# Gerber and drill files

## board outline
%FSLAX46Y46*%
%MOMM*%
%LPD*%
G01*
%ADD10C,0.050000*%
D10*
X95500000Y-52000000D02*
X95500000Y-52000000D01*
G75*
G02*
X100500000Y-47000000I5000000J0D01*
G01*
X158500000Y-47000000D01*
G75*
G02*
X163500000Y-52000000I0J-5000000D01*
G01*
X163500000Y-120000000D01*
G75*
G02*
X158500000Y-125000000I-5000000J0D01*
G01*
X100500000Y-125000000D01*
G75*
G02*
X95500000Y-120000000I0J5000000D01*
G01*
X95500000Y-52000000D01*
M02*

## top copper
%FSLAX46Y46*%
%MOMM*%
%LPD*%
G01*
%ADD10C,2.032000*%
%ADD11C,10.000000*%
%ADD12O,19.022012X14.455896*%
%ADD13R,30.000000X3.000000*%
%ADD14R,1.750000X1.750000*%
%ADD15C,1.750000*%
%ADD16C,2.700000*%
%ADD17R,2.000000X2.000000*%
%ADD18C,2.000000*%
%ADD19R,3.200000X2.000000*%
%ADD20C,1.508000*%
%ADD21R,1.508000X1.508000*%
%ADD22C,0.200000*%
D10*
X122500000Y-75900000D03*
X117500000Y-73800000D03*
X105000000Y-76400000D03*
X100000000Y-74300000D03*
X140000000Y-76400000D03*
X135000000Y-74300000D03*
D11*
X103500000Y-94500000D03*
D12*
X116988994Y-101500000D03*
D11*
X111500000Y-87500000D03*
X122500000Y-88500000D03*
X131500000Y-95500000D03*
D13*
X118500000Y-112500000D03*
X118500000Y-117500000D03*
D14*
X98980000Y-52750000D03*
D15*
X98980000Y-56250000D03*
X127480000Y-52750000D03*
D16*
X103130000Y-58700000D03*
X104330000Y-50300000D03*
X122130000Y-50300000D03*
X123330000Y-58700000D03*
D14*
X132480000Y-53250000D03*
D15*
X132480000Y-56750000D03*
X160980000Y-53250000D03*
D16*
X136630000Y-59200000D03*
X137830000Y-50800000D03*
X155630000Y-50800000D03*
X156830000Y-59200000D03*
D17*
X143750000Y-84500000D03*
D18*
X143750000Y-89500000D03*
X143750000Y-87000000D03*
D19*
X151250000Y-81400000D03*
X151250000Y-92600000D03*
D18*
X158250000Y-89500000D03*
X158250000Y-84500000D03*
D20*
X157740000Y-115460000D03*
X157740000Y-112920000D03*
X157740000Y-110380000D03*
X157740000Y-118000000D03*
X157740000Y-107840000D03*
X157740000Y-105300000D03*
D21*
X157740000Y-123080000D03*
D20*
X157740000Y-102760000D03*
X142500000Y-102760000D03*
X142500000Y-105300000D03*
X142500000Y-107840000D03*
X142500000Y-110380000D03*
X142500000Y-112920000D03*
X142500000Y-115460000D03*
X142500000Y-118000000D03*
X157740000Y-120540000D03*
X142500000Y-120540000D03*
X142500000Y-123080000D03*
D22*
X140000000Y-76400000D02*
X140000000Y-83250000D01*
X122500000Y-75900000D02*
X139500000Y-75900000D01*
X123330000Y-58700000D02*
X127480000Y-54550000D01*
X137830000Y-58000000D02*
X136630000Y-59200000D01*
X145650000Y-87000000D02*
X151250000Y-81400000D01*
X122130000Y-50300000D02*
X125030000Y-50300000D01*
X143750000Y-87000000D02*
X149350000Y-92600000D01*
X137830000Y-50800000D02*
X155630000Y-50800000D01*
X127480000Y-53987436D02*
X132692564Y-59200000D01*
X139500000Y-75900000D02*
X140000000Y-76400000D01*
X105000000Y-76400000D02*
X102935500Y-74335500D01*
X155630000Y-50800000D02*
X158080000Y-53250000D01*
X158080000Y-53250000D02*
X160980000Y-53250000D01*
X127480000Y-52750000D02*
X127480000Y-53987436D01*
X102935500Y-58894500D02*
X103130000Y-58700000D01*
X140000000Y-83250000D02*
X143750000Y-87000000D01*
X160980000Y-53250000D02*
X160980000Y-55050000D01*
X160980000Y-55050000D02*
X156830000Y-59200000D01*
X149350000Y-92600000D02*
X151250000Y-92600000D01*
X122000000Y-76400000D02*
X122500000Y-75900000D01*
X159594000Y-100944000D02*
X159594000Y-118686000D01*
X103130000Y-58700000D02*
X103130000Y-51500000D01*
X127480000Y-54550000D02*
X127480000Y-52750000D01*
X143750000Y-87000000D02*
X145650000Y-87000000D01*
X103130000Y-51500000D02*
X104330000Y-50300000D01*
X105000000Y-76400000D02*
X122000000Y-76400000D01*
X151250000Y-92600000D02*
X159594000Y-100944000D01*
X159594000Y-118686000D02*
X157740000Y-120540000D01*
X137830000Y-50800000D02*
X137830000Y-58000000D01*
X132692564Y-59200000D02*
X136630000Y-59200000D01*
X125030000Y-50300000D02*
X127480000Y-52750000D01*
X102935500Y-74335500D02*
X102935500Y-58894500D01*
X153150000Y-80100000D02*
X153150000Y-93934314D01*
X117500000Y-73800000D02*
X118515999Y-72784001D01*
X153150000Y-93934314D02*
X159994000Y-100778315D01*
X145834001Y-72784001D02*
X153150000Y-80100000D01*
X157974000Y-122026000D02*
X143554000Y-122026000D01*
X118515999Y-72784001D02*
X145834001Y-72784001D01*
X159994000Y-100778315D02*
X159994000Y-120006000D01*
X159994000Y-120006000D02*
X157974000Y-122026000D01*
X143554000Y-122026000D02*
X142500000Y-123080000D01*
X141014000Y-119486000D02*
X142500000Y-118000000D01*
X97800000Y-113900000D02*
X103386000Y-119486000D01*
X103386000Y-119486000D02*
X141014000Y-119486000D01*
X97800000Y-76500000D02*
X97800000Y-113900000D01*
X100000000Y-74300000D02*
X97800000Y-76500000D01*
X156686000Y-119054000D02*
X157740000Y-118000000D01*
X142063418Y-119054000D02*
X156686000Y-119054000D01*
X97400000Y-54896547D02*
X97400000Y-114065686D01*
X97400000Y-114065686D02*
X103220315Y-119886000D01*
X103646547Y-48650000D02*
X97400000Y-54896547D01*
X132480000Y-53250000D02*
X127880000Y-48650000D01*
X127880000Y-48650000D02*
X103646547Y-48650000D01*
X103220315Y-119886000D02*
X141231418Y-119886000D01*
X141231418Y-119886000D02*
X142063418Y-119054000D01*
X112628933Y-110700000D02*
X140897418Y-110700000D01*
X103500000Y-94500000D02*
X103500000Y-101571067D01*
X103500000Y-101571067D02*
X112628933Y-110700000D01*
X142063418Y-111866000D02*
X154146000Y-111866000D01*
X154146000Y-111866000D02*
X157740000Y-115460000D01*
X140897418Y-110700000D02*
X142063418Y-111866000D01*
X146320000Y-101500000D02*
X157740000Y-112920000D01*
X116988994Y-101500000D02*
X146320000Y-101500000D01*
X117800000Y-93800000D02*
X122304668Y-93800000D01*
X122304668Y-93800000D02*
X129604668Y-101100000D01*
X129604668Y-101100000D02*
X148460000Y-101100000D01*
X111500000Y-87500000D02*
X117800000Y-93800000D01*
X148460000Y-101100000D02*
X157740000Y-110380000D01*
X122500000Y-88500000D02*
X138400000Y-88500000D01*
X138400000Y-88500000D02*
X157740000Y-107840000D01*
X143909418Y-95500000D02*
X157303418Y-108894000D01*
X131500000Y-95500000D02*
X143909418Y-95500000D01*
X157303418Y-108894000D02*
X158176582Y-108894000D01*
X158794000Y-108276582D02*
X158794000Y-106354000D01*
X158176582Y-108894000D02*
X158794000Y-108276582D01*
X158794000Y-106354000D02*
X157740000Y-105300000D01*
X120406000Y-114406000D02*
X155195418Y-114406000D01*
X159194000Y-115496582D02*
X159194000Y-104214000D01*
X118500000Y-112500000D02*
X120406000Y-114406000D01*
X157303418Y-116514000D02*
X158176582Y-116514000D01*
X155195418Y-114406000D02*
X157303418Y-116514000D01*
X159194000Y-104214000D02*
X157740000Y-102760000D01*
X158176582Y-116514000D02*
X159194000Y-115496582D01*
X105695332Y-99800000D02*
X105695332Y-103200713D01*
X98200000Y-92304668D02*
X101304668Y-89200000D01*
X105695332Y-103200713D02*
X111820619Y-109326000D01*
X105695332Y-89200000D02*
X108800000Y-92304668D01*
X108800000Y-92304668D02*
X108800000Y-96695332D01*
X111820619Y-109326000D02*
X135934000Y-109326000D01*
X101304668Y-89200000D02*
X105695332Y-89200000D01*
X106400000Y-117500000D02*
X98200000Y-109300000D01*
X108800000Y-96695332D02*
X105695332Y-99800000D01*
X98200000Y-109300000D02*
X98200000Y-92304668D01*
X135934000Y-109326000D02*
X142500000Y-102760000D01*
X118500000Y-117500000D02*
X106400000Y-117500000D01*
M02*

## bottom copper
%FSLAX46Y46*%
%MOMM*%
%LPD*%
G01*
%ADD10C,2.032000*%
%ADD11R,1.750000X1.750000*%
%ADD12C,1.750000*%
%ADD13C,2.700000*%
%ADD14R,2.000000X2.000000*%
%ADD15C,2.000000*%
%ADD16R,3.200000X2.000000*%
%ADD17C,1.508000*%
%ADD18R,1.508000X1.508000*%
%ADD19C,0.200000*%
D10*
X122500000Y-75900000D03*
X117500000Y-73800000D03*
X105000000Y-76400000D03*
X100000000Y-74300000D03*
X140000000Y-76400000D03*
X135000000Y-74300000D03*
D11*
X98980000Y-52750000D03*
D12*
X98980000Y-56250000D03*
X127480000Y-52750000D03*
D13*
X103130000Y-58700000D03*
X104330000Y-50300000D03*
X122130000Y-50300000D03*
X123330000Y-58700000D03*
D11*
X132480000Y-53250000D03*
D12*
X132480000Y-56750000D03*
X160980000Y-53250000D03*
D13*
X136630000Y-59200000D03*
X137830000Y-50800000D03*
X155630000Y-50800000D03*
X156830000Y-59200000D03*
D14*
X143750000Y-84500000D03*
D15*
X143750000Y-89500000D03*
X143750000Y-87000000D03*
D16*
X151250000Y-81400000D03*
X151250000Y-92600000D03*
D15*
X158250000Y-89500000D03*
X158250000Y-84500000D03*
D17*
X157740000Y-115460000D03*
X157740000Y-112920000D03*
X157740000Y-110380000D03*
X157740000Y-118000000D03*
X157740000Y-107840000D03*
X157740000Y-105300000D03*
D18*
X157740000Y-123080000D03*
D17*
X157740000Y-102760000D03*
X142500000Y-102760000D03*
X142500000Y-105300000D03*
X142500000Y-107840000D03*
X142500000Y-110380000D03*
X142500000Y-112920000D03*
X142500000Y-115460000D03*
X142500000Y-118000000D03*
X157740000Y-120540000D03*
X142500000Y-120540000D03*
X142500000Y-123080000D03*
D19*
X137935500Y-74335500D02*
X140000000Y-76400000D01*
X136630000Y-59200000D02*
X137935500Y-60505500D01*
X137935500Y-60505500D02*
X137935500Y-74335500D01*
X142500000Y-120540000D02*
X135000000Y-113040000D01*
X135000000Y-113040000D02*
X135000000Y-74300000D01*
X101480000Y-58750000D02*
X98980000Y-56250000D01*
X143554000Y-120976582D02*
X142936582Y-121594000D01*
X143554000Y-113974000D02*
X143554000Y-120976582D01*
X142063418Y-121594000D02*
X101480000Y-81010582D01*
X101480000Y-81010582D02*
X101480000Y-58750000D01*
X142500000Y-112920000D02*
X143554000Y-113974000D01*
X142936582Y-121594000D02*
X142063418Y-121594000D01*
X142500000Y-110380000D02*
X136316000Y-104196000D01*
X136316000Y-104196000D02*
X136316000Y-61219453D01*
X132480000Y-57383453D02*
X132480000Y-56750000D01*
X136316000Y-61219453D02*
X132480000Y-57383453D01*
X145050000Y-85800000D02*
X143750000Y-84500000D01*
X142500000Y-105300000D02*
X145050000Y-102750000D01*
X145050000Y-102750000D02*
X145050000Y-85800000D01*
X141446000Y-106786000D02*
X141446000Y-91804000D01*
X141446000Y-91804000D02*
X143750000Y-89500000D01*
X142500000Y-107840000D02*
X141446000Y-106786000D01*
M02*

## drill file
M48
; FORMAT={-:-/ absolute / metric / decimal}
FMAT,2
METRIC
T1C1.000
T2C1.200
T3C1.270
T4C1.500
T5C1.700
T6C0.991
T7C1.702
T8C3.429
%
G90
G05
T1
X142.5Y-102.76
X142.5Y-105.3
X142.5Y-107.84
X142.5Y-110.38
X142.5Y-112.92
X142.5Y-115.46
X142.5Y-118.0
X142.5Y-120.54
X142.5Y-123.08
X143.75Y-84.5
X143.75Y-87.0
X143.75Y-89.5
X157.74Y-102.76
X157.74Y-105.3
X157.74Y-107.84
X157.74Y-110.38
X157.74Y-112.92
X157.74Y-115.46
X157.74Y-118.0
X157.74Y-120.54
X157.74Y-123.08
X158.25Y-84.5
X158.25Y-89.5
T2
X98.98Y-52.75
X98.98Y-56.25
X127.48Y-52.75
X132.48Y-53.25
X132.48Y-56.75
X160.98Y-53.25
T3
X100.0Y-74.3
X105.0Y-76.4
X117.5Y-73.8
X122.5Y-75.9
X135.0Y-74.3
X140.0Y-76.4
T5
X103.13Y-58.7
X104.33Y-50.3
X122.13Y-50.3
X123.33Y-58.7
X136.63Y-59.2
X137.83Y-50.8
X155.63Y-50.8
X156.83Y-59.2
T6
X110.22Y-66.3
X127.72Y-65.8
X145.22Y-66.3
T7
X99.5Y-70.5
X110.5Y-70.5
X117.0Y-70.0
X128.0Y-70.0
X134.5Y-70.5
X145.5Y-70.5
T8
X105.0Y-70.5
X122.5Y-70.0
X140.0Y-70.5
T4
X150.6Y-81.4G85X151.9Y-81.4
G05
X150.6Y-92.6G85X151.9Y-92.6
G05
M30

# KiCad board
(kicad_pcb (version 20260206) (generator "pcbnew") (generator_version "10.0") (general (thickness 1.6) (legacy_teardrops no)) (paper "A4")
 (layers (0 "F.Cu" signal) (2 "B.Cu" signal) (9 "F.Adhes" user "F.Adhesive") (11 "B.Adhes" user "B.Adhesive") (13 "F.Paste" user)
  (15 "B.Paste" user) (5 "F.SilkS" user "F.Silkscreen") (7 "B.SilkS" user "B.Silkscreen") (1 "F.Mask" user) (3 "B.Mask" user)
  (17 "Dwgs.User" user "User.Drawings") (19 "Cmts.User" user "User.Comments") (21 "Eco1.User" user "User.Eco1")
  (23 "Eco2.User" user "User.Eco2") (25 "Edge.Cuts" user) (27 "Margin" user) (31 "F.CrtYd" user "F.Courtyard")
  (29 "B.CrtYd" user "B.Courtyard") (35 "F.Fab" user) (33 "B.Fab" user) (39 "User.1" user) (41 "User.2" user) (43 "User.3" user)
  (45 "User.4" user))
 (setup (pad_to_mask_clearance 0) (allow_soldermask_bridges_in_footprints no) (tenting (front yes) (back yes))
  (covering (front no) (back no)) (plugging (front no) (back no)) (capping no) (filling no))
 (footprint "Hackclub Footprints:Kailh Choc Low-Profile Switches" (layer "F.Cu") (at 122.5 70)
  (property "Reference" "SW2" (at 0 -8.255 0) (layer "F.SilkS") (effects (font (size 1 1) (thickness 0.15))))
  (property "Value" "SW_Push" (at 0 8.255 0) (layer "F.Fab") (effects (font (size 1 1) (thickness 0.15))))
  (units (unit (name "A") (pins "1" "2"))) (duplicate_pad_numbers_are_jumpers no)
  (pad "" np_thru_hole circle (at -5.5 0) (size 1.7018 1.7018) (drill 1.7018) (layers "*.Cu" "*.Mask"))
  (pad "" np_thru_hole circle (at 0 0) (size 3.429 3.429) (drill 3.429) (layers "*.Cu" "*.Mask"))
  (pad "" np_thru_hole circle (at 5.22 -4.2) (size 0.9906 0.9906) (drill 0.9906) (layers "*.Cu" "*.Mask"))
  (pad "" np_thru_hole circle (at 5.5 0) (size 1.7018 1.7018) (drill 1.7018) (layers "*.Cu" "*.Mask"))
  (pad "1" thru_hole circle (at 0 5.9) (size 2.032 2.032) (drill 1.27) (layers "*.Cu" "*.Mask") (remove_unused_layers no) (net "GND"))
  (pad "2" thru_hole circle (at -5 3.8) (size 2.032 2.032) (drill 1.27) (layers "*.Cu" "*.Mask") (remove_unused_layers no) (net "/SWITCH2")))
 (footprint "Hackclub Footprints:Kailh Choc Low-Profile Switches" (layer "F.Cu") (at 105 70.5)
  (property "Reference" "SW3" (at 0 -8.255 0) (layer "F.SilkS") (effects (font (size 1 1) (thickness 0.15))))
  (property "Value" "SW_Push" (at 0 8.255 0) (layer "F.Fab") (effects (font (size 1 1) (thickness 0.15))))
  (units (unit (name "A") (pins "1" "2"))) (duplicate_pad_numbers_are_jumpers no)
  (pad "" np_thru_hole circle (at -5.5 0) (size 1.7018 1.7018) (drill 1.7018) (layers "*.Cu" "*.Mask"))
  (pad "" np_thru_hole circle (at 0 0) (size 3.429 3.429) (drill 3.429) (layers "*.Cu" "*.Mask"))
  (pad "" np_thru_hole circle (at 5.22 -4.2) (size 0.9906 0.9906) (drill 0.9906) (layers "*.Cu" "*.Mask"))
  (pad "" np_thru_hole circle (at 5.5 0) (size 1.7018 1.7018) (drill 1.7018) (layers "*.Cu" "*.Mask"))
  (pad "1" thru_hole circle (at 0 5.9) (size 2.032 2.032) (drill 1.27) (layers "*.Cu" "*.Mask") (remove_unused_layers no) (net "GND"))
  (pad "2" thru_hole circle (at -5 3.8) (size 2.032 2.032) (drill 1.27) (layers "*.Cu" "*.Mask") (remove_unused_layers no) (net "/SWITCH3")))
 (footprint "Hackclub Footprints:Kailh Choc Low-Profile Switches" (layer "F.Cu") (at 140 70.5)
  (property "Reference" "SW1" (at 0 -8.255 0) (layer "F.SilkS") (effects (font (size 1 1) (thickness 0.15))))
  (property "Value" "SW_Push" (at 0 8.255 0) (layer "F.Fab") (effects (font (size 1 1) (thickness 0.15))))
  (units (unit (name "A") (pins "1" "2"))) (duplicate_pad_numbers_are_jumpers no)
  (pad "" np_thru_hole circle (at -5.5 0) (size 1.7018 1.7018) (drill 1.7018) (layers "*.Cu" "*.Mask"))
  (pad "" np_thru_hole circle (at 0 0) (size 3.429 3.429) (drill 3.429) (layers "*.Cu" "*.Mask"))
  (pad "" np_thru_hole circle (at 5.22 -4.2) (size 0.9906 0.9906) (drill 0.9906) (layers "*.Cu" "*.Mask"))
  (pad "" np_thru_hole circle (at 5.5 0) (size 1.7018 1.7018) (drill 1.7018) (layers "*.Cu" "*.Mask"))
  (pad "1" thru_hole circle (at 0 5.9) (size 2.032 2.032) (drill 1.27) (layers "*.Cu" "*.Mask") (remove_unused_layers no) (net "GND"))
  (pad "2" thru_hole circle (at -5 3.8) (size 2.032 2.032) (drill 1.27) (layers "*.Cu" "*.Mask") (remove_unused_layers no) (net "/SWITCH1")))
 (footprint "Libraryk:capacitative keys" (layer "F.Cu") (at 102.5 54.5)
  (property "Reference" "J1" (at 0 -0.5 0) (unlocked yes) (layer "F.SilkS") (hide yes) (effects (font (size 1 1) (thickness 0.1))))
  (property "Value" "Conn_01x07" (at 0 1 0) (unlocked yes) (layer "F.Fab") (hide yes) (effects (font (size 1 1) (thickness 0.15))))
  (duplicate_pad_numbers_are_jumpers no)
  (pad "1" smd circle (at 1 40) (size 10 10) (layers "F.Cu" "F.Mask") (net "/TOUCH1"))
  (pad "2" smd oval (at 14.488994 47 90) (size 14.455896 19.022012) (layers "F.Cu" "F.Mask") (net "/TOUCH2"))
  (pad "3" smd circle (at 9 33) (size 10 10) (layers "F.Cu" "F.Mask") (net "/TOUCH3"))
  (pad "4" smd circle (at 20 34) (size 10 10) (layers "F.Cu" "F.Mask") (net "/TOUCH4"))
  (pad "5" smd circle (at 29 41) (size 10 10) (layers "F.Cu" "F.Mask") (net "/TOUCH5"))
  (pad "6" smd rect (at 16 58) (size 30 3) (layers "F.Cu" "F.Mask") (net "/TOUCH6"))
  (pad "7" smd rect (at 16 63) (size 30 3) (layers "F.Cu" "F.Mask") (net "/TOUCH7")))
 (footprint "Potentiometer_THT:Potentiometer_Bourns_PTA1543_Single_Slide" (layer "F.Cu") (at 98.98 52.75)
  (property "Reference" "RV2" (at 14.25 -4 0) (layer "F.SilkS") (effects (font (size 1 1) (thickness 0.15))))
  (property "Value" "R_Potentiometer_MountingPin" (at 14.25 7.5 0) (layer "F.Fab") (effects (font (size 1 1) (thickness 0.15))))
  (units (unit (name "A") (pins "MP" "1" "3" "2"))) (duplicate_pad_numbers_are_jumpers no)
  (pad "1" thru_hole rect (at 0 0) (size 1.75 1.75) (drill 1.2) (layers "*.Cu" "*.Mask") (remove_unused_layers no) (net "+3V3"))
  (pad "2" thru_hole circle (at 0 3.5) (size 1.75 1.75) (drill 1.2) (layers "*.Cu" "*.Mask") (remove_unused_layers no) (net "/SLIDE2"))
  (pad "3" thru_hole circle (at 28.5 0) (size 1.75 1.75) (drill 1.2) (layers "*.Cu" "*.Mask") (remove_unused_layers no) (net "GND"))
  (pad "MP" thru_hole circle (at 4.15 5.95) (size 2.7 2.7) (drill 1.7) (layers "*.Cu" "*.Mask") (remove_unused_layers no) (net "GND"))
  (pad "MP" thru_hole circle (at 5.35 -2.45) (size 2.7 2.7) (drill 1.7) (layers "*.Cu" "*.Mask") (remove_unused_layers no) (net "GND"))
  (pad "MP" thru_hole circle (at 23.15 -2.45) (size 2.7 2.7) (drill 1.7) (layers "*.Cu" "*.Mask") (remove_unused_layers no) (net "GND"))
  (pad "MP" thru_hole circle (at 24.35 5.95) (size 2.7 2.7) (drill 1.7) (layers "*.Cu" "*.Mask") (remove_unused_layers no) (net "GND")))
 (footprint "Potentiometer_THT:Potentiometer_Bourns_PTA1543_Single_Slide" (layer "F.Cu") (at 132.48 53.25)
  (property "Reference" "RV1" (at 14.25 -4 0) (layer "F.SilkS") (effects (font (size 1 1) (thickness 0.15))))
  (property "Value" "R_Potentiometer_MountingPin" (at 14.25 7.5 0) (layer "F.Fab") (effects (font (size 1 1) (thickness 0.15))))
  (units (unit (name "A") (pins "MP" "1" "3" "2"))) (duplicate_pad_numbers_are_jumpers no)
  (pad "1" thru_hole rect (at 0 0) (size 1.75 1.75) (drill 1.2) (layers "*.Cu" "*.Mask") (remove_unused_layers no) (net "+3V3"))
  (pad "2" thru_hole circle (at 0 3.5) (size 1.75 1.75) (drill 1.2) (layers "*.Cu" "*.Mask") (remove_unused_layers no) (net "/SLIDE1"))
  (pad "3" thru_hole circle (at 28.5 0) (size 1.75 1.75) (drill 1.2) (layers "*.Cu" "*.Mask") (remove_unused_layers no) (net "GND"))
  (pad "MP" thru_hole circle (at 4.15 5.95) (size 2.7 2.7) (drill 1.7) (layers "*.Cu" "*.Mask") (remove_unused_layers no) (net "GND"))
  (pad "MP" thru_hole circle (at 5.35 -2.45) (size 2.7 2.7) (drill 1.7) (layers "*.Cu" "*.Mask") (remove_unused_layers no) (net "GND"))
  (pad "MP" thru_hole circle (at 23.15 -2.45) (size 2.7 2.7) (drill 1.7) (layers "*.Cu" "*.Mask") (remove_unused_layers no) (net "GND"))
  (pad "MP" thru_hole circle (at 24.35 5.95) (size 2.7 2.7) (drill 1.7) (layers "*.Cu" "*.Mask") (remove_unused_layers no) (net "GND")))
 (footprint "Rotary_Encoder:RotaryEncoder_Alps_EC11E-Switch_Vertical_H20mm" (layer "F.Cu") (at 143.75 84.5)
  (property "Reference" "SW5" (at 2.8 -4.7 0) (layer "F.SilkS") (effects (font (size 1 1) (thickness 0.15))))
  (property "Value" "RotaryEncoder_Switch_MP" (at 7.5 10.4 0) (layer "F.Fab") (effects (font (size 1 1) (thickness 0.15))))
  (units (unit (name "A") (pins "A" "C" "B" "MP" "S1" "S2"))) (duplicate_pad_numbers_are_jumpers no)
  (pad "A" thru_hole rect (at 0 0) (size 2 2) (drill 1) (layers "*.Cu" "*.Mask") (remove_unused_layers no) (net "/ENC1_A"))
  (pad "B" thru_hole circle (at 0 5) (size 2 2) (drill 1) (layers "*.Cu" "*.Mask") (remove_unused_layers no) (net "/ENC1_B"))
  (pad "C" thru_hole circle (at 0 2.5) (size 2 2) (drill 1) (layers "*.Cu" "*.Mask") (remove_unused_layers no) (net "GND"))
  (pad "MP" thru_hole rect (at 7.5 -3.1) (size 3.2 2) (drill oval 2.8 1.5) (layers "*.Cu" "*.Mask") (remove_unused_layers no) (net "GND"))
  (pad "MP" thru_hole rect (at 7.5 8.1) (size 3.2 2) (drill oval 2.8 1.5) (layers "*.Cu" "*.Mask") (remove_unused_layers no) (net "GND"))
  (pad "S1" thru_hole circle (at 14.5 5) (size 2 2) (drill 1) (layers "*.Cu" "*.Mask") (remove_unused_layers no)
   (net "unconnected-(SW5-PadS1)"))
  (pad "S2" thru_hole circle (at 14.5 0) (size 2 2) (drill 1) (layers "*.Cu" "*.Mask") (remove_unused_layers no)
   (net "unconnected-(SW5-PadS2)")))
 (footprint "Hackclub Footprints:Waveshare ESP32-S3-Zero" (layer "F.Cu") (at 150.12 112.92 180)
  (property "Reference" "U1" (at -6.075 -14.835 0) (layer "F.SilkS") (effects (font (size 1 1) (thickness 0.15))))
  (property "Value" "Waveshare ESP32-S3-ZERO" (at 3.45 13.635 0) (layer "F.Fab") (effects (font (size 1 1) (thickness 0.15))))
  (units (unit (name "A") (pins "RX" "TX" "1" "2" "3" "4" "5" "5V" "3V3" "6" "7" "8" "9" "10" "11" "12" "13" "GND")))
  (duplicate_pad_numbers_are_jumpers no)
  (pad "1" thru_hole circle (at -7.62 -2.54 180) (size 1.508 1.508) (drill 1) (layers "*.Cu" "*.Mask") (remove_unused_layers no)
   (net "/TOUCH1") (solder_mask_margin 0.102))
  (pad "2" thru_hole circle (at -7.62 0 180) (size 1.508 1.508) (drill 1) (layers "*.Cu" "*.Mask") (remove_unused_layers no) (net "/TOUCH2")
   (solder_mask_margin 0.102))
  (pad "3" thru_hole circle (at -7.62 2.54 180) (size 1.508 1.508) (drill 1) (layers "*.Cu" "*.Mask") (remove_unused_layers no)
   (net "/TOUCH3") (solder_mask_margin 0.102))
  (pad "3V3" thru_hole circle (at -7.62 -5.08 180) (size 1.508 1.508) (drill 1) (layers "*.Cu" "*.Mask") (remove_unused_layers no)
   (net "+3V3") (solder_mask_margin 0.102))
  (pad "4" thru_hole circle (at -7.62 5.08 180) (size 1.508 1.508) (drill 1) (layers "*.Cu" "*.Mask") (remove_unused_layers no)
   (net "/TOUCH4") (solder_mask_margin 0.102))
  (pad "5" thru_hole circle (at -7.62 7.62 180) (size 1.508 1.508) (drill 1) (layers "*.Cu" "*.Mask") (remove_unused_layers no)
   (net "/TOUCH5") (solder_mask_margin 0.102))
  (pad "5V" thru_hole rect (at -7.62 -10.16 180) (size 1.508 1.508) (drill 1) (layers "*.Cu" "*.Mask") (remove_unused_layers no) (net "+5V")
   (solder_mask_margin 0.102))
  (pad "6" thru_hole circle (at -7.62 10.16 180) (size 1.508 1.508) (drill 1) (layers "*.Cu" "*.Mask") (remove_unused_layers no)
   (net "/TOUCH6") (solder_mask_margin 0.102))
  (pad "7" thru_hole circle (at 7.62 10.16 180) (size 1.508 1.508) (drill 1) (layers "*.Cu" "*.Mask") (remove_unused_layers no)
   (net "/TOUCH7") (solder_mask_margin 0.102))
  (pad "8" thru_hole circle (at 7.62 7.62 180) (size 1.508 1.508) (drill 1) (layers "*.Cu" "*.Mask") (remove_unused_layers no)
   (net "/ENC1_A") (solder_mask_margin 0.102))
  (pad "9" thru_hole circle (at 7.62 5.08 180) (size 1.508 1.508) (drill 1) (layers "*.Cu" "*.Mask") (remove_unused_layers no)
   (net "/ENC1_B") (solder_mask_margin 0.102))
  (pad "10" thru_hole circle (at 7.62 2.54 180) (size 1.508 1.508) (drill 1) (layers "*.Cu" "*.Mask") (remove_unused_layers no)
   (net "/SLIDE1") (solder_mask_margin 0.102))
  (pad "11" thru_hole circle (at 7.62 0 180) (size 1.508 1.508) (drill 1) (layers "*.Cu" "*.Mask") (remove_unused_layers no) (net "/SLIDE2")
   (solder_mask_margin 0.102))
  (pad "12" thru_hole circle (at 7.62 -2.54 180) (size 1.508 1.508) (drill 1) (layers "*.Cu" "*.Mask") (remove_unused_layers no)
   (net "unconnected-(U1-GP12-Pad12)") (solder_mask_margin 0.102))
  (pad "13" thru_hole circle (at 7.62 -5.08 180) (size 1.508 1.508) (drill 1) (layers "*.Cu" "*.Mask") (remove_unused_layers no)
   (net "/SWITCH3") (solder_mask_margin 0.102))
  (pad "GND" thru_hole circle (at -7.62 -7.62 180) (size 1.508 1.508) (drill 1) (layers "*.Cu" "*.Mask") (remove_unused_layers no)
   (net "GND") (solder_mask_margin 0.102))
  (pad "RX" thru_hole circle (at 7.62 -7.62 180) (size 1.508 1.508) (drill 1) (layers "*.Cu" "*.Mask") (remove_unused_layers no)
   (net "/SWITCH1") (solder_mask_margin 0.102))
  (pad "TX" thru_hole circle (at 7.62 -10.16 180) (size 1.508 1.508) (drill 1) (layers "*.Cu" "*.Mask") (remove_unused_layers no)
   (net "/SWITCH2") (solder_mask_margin 0.102)))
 (gr_rect (start 95.5 47) (end 163.5 125) (radius 5) (stroke (width 0.05) (type solid)) (fill no) (layer "Edge.Cuts"))
 (segment (start 140 76.4) (end 140 83.25) (width 0.2) (layer "F.Cu") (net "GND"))
 (segment (start 122.5 75.9) (end 139.5 75.9) (width 0.2) (layer "F.Cu") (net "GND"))
 (segment (start 123.33 58.7) (end 127.48 54.55) (width 0.2) (layer "F.Cu") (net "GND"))
 (segment (start 137.83 58) (end 136.63 59.2) (width 0.2) (layer "F.Cu") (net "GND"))
 (segment (start 145.65 87) (end 151.25 81.4) (width 0.2) (layer "F.Cu") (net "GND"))
 (segment (start 122.13 50.3) (end 125.03 50.3) (width 0.2) (layer "F.Cu") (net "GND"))
 (segment (start 143.75 87) (end 149.35 92.6) (width 0.2) (layer "F.Cu") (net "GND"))
 (segment (start 137.83 50.8) (end 155.63 50.8) (width 0.2) (layer "F.Cu") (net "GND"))
 (segment (start 127.48 53.987436) (end 132.692564 59.2) (width 0.2) (layer "F.Cu") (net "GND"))
 (segment (start 139.5 75.9) (end 140 76.4) (width 0.2) (layer "F.Cu") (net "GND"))
 (segment (start 105 76.4) (end 102.9355 74.3355) (width 0.2) (layer "F.Cu") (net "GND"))
 (segment (start 155.63 50.8) (end 158.08 53.25) (width 0.2) (layer "F.Cu") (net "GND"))
 (segment (start 158.08 53.25) (end 160.98 53.25) (width 0.2) (layer "F.Cu") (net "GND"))
 (segment (start 127.48 52.75) (end 127.48 53.987436) (width 0.2) (layer "F.Cu") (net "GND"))
 (segment (start 102.9355 58.8945) (end 103.13 58.7) (width 0.2) (layer "F.Cu") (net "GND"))
 (segment (start 140 83.25) (end 143.75 87) (width 0.2) (layer "F.Cu") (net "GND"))
 (segment (start 160.98 53.25) (end 160.98 55.05) (width 0.2) (layer "F.Cu") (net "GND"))
 (segment (start 160.98 55.05) (end 156.83 59.2) (width 0.2) (layer "F.Cu") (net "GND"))
 (segment (start 149.35 92.6) (end 151.25 92.6) (width 0.2) (layer "F.Cu") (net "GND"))
 (segment (start 122 76.4) (end 122.5 75.9) (width 0.2) (layer "F.Cu") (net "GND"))
 (segment (start 159.594 100.944) (end 159.594 118.686) (width 0.2) (layer "F.Cu") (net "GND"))
 (segment (start 103.13 58.7) (end 103.13 51.5) (width 0.2) (layer "F.Cu") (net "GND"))
 (segment (start 127.48 54.55) (end 127.48 52.75) (width 0.2) (layer "F.Cu") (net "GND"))
 (segment (start 143.75 87) (end 145.65 87) (width 0.2) (layer "F.Cu") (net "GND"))
 (segment (start 103.13 51.5) (end 104.33 50.3) (width 0.2) (layer "F.Cu") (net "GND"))
 (segment (start 105 76.4) (end 122 76.4) (width 0.2) (layer "F.Cu") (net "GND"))
 (segment (start 151.25 92.6) (end 159.594 100.944) (width 0.2) (layer "F.Cu") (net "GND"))
 (segment (start 159.594 118.686) (end 157.74 120.54) (width 0.2) (layer "F.Cu") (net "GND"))
 (segment (start 137.83 50.8) (end 137.83 58) (width 0.2) (layer "F.Cu") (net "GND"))
 (segment (start 132.692564 59.2) (end 136.63 59.2) (width 0.2) (layer "F.Cu") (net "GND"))
 (segment (start 125.03 50.3) (end 127.48 52.75) (width 0.2) (layer "F.Cu") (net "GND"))
 (segment (start 102.9355 74.3355) (end 102.9355 58.8945) (width 0.2) (layer "F.Cu") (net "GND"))
 (segment (start 137.9355 74.3355) (end 140 76.4) (width 0.2) (layer "B.Cu") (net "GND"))
 (segment (start 136.63 59.2) (end 137.9355 60.5055) (width 0.2) (layer "B.Cu") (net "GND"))
 (segment (start 137.9355 60.5055) (end 137.9355 74.3355) (width 0.2) (layer "B.Cu") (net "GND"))
 (segment (start 153.15 80.1) (end 153.15 93.934314) (width 0.2) (layer "F.Cu") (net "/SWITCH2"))
 (segment (start 117.5 73.8) (end 118.515999 72.784001) (width 0.2) (layer "F.Cu") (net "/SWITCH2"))
 (segment (start 153.15 93.934314) (end 159.994 100.778315) (width 0.2) (layer "F.Cu") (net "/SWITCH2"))
 (segment (start 145.834001 72.784001) (end 153.15 80.1) (width 0.2) (layer "F.Cu") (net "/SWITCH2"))
 (segment (start 157.974 122.026) (end 143.554 122.026) (width 0.2) (layer "F.Cu") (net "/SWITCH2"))
 (segment (start 118.515999 72.784001) (end 145.834001 72.784001) (width 0.2) (layer "F.Cu") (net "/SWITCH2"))
 (segment (start 159.994 100.778315) (end 159.994 120.006) (width 0.2) (layer "F.Cu") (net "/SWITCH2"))
 (segment (start 159.994 120.006) (end 157.974 122.026) (width 0.2) (layer "F.Cu") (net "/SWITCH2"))
 (segment (start 143.554 122.026) (end 142.5 123.08) (width 0.2) (layer "F.Cu") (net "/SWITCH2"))
 (segment (start 141.014 119.486) (end 142.5 118) (width 0.2) (layer "F.Cu") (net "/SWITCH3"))
 (segment (start 97.8 113.9) (end 103.386 119.486) (width 0.2) (layer "F.Cu") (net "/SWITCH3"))
 (segment (start 103.386 119.486) (end 141.014 119.486) (width 0.2) (layer "F.Cu") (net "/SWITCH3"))
 (segment (start 97.8 76.5) (end 97.8 113.9) (width 0.2) (layer "F.Cu") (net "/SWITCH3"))
 (segment (start 100 74.3) (end 97.8 76.5) (width 0.2) (layer "F.Cu") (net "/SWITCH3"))
 (segment (start 142.5 120.54) (end 135 113.04) (width 0.2) (layer "B.Cu") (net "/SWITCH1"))
 (segment (start 135 113.04) (end 135 74.3) (width 0.2) (layer "B.Cu") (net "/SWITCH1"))
 (segment (start 156.686 119.054) (end 157.74 118) (width 0.2) (layer "F.Cu") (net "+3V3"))
 (segment (start 142.063418 119.054) (end 156.686 119.054) (width 0.2) (layer "F.Cu") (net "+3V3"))
 (segment (start 97.4 54.896547) (end 97.4 114.065686) (width 0.2) (layer "F.Cu") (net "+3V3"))
 (segment (start 97.4 114.065686) (end 103.220315 119.886) (width 0.2) (layer "F.Cu") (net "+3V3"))
 (segment (start 103.646547 48.65) (end 97.4 54.896547) (width 0.2) (layer "F.Cu") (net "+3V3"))
 (segment (start 132.48 53.25) (end 127.88 48.65) (width 0.2) (layer "F.Cu") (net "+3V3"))
 (segment (start 127.88 48.65) (end 103.646547 48.65) (width 0.2) (layer "F.Cu") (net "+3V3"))
 (segment (start 103.220315 119.886) (end 141.231418 119.886) (width 0.2) (layer "F.Cu") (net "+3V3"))
 (segment (start 141.231418 119.886) (end 142.063418 119.054) (width 0.2) (layer "F.Cu") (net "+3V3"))
 (segment (start 101.48 58.75) (end 98.98 56.25) (width 0.2) (layer "B.Cu") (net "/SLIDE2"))
 (segment (start 143.554 120.976582) (end 142.936582 121.594) (width 0.2) (layer "B.Cu") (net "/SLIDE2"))
 (segment (start 143.554 113.974) (end 143.554 120.976582) (width 0.2) (layer "B.Cu") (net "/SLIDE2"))
 (segment (start 142.063418 121.594) (end 101.48 81.010582) (width 0.2) (layer "B.Cu") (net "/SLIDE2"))
 (segment (start 101.48 81.010582) (end 101.48 58.75) (width 0.2) (layer "B.Cu") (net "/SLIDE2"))
 (segment (start 142.5 112.92) (end 143.554 113.974) (width 0.2) (layer "B.Cu") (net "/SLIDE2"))
 (segment (start 142.936582 121.594) (end 142.063418 121.594) (width 0.2) (layer "B.Cu") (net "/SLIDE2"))
 (segment (start 142.5 110.38) (end 136.316 104.196) (width 0.2) (layer "B.Cu") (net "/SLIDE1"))
 (segment (start 136.316 104.196) (end 136.316 61.219453) (width 0.2) (layer "B.Cu") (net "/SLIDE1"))
 (segment (start 132.48 57.383453) (end 132.48 56.75) (width 0.2) (layer "B.Cu") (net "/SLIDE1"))
 (segment (start 136.316 61.219453) (end 132.48 57.383453) (width 0.2) (layer "B.Cu") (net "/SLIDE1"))
 (segment (start 145.05 85.8) (end 143.75 84.5) (width 0.2) (layer "B.Cu") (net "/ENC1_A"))
 (segment (start 142.5 105.3) (end 145.05 102.75) (width 0.2) (layer "B.Cu") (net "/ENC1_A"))
 (segment (start 145.05 102.75) (end 145.05 85.8) (width 0.2) (layer "B.Cu") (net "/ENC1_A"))
 (segment (start 141.446 106.786) (end 141.446 91.804) (width 0.2) (layer "B.Cu") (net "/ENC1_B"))
 (segment (start 141.446 91.804) (end 143.75 89.5) (width 0.2) (layer "B.Cu") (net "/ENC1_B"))
 (segment (start 142.5 107.84) (end 141.446 106.786) (width 0.2) (layer "B.Cu") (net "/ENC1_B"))
 (segment (start 112.628933 110.7) (end 140.897418 110.7) (width 0.2) (layer "F.Cu") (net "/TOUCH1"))
 (segment (start 103.5 94.5) (end 103.5 101.571067) (width 0.2) (layer "F.Cu") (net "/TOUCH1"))
 (segment (start 103.5 101.571067) (end 112.628933 110.7) (width 0.2) (layer "F.Cu") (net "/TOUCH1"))
 (segment (start 142.063418 111.866) (end 154.146 111.866) (width 0.2) (layer "F.Cu") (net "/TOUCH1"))
 (segment (start 154.146 111.866) (end 157.74 115.46) (width 0.2) (layer "F.Cu") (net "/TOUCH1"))
 (segment (start 140.897418 110.7) (end 142.063418 111.866) (width 0.2) (layer "F.Cu") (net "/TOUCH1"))
 (segment (start 146.32 101.5) (end 157.74 112.92) (width 0.2) (layer "F.Cu") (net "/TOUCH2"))
 (segment (start 116.988994 101.5) (end 146.32 101.5) (width 0.2) (layer "F.Cu") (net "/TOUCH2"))
 (segment (start 117.8 93.8) (end 122.304668 93.8) (width 0.2) (layer "F.Cu") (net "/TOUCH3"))
 (segment (start 122.304668 93.8) (end 129.604668 101.1) (width 0.2) (layer "F.Cu") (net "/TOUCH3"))
 (segment (start 129.604668 101.1) (end 148.46 101.1) (width 0.2) (layer "F.Cu") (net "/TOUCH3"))
 (segment (start 111.5 87.5) (end 117.8 93.8) (width 0.2) (layer "F.Cu") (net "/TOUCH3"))
 (segment (start 148.46 101.1) (end 157.74 110.38) (width 0.2) (layer "F.Cu") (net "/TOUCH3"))
 (segment (start 122.5 88.5) (end 138.4 88.5) (width 0.2) (layer "F.Cu") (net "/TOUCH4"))
 (segment (start 138.4 88.5) (end 157.74 107.84) (width 0.2) (layer "F.Cu") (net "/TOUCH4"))
 (segment (start 143.909418 95.5) (end 157.303418 108.894) (width 0.2) (layer "F.Cu") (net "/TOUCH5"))
 (segment (start 131.5 95.5) (end 143.909418 95.5) (width 0.2) (layer "F.Cu") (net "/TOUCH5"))
 (segment (start 157.303418 108.894) (end 158.176582 108.894) (width 0.2) (layer "F.Cu") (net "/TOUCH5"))
 (segment (start 158.794 108.276582) (end 158.794 106.354) (width 0.2) (layer "F.Cu") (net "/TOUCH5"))
 (segment (start 158.176582 108.894) (end 158.794 108.276582) (width 0.2) (layer "F.Cu") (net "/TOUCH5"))
 (segment (start 158.794 106.354) (end 157.74 105.3) (width 0.2) (layer "F.Cu") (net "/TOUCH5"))
 (segment (start 120.406 114.406) (end 155.195418 114.406) (width 0.2) (layer "F.Cu") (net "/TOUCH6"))
 (segment (start 159.194 115.496582) (end 159.194 104.214) (width 0.2) (layer "F.Cu") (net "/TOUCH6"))
 (segment (start 118.5 112.5) (end 120.406 114.406) (width 0.2) (layer "F.Cu") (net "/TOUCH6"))
 (segment (start 157.303418 116.514) (end 158.176582 116.514) (width 0.2) (layer "F.Cu") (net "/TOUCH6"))
 (segment (start 155.195418 114.406) (end 157.303418 116.514) (width 0.2) (layer "F.Cu") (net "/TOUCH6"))
 (segment (start 159.194 104.214) (end 157.74 102.76) (width 0.2) (layer "F.Cu") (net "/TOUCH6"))
 (segment (start 158.176582 116.514) (end 159.194 115.496582) (width 0.2) (layer "F.Cu") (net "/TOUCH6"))
 (segment (start 105.695332 99.8) (end 105.695332 103.200713) (width 0.2) (layer "F.Cu") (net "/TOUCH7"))
 (segment (start 98.2 92.304668) (end 101.304668 89.2) (width 0.2) (layer "F.Cu") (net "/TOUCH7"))
 (segment (start 105.695332 103.200713) (end 111.820619 109.326) (width 0.2) (layer "F.Cu") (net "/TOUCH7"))
 (segment (start 105.695332 89.2) (end 108.8 92.304668) (width 0.2) (layer "F.Cu") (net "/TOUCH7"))
 (segment (start 108.8 92.304668) (end 108.8 96.695332) (width 0.2) (layer "F.Cu") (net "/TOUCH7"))
 (segment (start 111.820619 109.326) (end 135.934 109.326) (width 0.2) (layer "F.Cu") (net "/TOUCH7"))
 (segment (start 101.304668 89.2) (end 105.695332 89.2) (width 0.2) (layer "F.Cu") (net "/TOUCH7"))
 (segment (start 106.4 117.5) (end 98.2 109.3) (width 0.2) (layer "F.Cu") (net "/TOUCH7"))
 (segment (start 108.8 96.695332) (end 105.695332 99.8) (width 0.2) (layer "F.Cu") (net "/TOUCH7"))
 (segment (start 98.2 109.3) (end 98.2 92.304668) (width 0.2) (layer "F.Cu") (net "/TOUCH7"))
 (segment (start 135.934 109.326) (end 142.5 102.76) (width 0.2) (layer "F.Cu") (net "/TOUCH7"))
 (segment (start 118.5 117.5) (end 106.4 117.5) (width 0.2) (layer "F.Cu") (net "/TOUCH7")))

